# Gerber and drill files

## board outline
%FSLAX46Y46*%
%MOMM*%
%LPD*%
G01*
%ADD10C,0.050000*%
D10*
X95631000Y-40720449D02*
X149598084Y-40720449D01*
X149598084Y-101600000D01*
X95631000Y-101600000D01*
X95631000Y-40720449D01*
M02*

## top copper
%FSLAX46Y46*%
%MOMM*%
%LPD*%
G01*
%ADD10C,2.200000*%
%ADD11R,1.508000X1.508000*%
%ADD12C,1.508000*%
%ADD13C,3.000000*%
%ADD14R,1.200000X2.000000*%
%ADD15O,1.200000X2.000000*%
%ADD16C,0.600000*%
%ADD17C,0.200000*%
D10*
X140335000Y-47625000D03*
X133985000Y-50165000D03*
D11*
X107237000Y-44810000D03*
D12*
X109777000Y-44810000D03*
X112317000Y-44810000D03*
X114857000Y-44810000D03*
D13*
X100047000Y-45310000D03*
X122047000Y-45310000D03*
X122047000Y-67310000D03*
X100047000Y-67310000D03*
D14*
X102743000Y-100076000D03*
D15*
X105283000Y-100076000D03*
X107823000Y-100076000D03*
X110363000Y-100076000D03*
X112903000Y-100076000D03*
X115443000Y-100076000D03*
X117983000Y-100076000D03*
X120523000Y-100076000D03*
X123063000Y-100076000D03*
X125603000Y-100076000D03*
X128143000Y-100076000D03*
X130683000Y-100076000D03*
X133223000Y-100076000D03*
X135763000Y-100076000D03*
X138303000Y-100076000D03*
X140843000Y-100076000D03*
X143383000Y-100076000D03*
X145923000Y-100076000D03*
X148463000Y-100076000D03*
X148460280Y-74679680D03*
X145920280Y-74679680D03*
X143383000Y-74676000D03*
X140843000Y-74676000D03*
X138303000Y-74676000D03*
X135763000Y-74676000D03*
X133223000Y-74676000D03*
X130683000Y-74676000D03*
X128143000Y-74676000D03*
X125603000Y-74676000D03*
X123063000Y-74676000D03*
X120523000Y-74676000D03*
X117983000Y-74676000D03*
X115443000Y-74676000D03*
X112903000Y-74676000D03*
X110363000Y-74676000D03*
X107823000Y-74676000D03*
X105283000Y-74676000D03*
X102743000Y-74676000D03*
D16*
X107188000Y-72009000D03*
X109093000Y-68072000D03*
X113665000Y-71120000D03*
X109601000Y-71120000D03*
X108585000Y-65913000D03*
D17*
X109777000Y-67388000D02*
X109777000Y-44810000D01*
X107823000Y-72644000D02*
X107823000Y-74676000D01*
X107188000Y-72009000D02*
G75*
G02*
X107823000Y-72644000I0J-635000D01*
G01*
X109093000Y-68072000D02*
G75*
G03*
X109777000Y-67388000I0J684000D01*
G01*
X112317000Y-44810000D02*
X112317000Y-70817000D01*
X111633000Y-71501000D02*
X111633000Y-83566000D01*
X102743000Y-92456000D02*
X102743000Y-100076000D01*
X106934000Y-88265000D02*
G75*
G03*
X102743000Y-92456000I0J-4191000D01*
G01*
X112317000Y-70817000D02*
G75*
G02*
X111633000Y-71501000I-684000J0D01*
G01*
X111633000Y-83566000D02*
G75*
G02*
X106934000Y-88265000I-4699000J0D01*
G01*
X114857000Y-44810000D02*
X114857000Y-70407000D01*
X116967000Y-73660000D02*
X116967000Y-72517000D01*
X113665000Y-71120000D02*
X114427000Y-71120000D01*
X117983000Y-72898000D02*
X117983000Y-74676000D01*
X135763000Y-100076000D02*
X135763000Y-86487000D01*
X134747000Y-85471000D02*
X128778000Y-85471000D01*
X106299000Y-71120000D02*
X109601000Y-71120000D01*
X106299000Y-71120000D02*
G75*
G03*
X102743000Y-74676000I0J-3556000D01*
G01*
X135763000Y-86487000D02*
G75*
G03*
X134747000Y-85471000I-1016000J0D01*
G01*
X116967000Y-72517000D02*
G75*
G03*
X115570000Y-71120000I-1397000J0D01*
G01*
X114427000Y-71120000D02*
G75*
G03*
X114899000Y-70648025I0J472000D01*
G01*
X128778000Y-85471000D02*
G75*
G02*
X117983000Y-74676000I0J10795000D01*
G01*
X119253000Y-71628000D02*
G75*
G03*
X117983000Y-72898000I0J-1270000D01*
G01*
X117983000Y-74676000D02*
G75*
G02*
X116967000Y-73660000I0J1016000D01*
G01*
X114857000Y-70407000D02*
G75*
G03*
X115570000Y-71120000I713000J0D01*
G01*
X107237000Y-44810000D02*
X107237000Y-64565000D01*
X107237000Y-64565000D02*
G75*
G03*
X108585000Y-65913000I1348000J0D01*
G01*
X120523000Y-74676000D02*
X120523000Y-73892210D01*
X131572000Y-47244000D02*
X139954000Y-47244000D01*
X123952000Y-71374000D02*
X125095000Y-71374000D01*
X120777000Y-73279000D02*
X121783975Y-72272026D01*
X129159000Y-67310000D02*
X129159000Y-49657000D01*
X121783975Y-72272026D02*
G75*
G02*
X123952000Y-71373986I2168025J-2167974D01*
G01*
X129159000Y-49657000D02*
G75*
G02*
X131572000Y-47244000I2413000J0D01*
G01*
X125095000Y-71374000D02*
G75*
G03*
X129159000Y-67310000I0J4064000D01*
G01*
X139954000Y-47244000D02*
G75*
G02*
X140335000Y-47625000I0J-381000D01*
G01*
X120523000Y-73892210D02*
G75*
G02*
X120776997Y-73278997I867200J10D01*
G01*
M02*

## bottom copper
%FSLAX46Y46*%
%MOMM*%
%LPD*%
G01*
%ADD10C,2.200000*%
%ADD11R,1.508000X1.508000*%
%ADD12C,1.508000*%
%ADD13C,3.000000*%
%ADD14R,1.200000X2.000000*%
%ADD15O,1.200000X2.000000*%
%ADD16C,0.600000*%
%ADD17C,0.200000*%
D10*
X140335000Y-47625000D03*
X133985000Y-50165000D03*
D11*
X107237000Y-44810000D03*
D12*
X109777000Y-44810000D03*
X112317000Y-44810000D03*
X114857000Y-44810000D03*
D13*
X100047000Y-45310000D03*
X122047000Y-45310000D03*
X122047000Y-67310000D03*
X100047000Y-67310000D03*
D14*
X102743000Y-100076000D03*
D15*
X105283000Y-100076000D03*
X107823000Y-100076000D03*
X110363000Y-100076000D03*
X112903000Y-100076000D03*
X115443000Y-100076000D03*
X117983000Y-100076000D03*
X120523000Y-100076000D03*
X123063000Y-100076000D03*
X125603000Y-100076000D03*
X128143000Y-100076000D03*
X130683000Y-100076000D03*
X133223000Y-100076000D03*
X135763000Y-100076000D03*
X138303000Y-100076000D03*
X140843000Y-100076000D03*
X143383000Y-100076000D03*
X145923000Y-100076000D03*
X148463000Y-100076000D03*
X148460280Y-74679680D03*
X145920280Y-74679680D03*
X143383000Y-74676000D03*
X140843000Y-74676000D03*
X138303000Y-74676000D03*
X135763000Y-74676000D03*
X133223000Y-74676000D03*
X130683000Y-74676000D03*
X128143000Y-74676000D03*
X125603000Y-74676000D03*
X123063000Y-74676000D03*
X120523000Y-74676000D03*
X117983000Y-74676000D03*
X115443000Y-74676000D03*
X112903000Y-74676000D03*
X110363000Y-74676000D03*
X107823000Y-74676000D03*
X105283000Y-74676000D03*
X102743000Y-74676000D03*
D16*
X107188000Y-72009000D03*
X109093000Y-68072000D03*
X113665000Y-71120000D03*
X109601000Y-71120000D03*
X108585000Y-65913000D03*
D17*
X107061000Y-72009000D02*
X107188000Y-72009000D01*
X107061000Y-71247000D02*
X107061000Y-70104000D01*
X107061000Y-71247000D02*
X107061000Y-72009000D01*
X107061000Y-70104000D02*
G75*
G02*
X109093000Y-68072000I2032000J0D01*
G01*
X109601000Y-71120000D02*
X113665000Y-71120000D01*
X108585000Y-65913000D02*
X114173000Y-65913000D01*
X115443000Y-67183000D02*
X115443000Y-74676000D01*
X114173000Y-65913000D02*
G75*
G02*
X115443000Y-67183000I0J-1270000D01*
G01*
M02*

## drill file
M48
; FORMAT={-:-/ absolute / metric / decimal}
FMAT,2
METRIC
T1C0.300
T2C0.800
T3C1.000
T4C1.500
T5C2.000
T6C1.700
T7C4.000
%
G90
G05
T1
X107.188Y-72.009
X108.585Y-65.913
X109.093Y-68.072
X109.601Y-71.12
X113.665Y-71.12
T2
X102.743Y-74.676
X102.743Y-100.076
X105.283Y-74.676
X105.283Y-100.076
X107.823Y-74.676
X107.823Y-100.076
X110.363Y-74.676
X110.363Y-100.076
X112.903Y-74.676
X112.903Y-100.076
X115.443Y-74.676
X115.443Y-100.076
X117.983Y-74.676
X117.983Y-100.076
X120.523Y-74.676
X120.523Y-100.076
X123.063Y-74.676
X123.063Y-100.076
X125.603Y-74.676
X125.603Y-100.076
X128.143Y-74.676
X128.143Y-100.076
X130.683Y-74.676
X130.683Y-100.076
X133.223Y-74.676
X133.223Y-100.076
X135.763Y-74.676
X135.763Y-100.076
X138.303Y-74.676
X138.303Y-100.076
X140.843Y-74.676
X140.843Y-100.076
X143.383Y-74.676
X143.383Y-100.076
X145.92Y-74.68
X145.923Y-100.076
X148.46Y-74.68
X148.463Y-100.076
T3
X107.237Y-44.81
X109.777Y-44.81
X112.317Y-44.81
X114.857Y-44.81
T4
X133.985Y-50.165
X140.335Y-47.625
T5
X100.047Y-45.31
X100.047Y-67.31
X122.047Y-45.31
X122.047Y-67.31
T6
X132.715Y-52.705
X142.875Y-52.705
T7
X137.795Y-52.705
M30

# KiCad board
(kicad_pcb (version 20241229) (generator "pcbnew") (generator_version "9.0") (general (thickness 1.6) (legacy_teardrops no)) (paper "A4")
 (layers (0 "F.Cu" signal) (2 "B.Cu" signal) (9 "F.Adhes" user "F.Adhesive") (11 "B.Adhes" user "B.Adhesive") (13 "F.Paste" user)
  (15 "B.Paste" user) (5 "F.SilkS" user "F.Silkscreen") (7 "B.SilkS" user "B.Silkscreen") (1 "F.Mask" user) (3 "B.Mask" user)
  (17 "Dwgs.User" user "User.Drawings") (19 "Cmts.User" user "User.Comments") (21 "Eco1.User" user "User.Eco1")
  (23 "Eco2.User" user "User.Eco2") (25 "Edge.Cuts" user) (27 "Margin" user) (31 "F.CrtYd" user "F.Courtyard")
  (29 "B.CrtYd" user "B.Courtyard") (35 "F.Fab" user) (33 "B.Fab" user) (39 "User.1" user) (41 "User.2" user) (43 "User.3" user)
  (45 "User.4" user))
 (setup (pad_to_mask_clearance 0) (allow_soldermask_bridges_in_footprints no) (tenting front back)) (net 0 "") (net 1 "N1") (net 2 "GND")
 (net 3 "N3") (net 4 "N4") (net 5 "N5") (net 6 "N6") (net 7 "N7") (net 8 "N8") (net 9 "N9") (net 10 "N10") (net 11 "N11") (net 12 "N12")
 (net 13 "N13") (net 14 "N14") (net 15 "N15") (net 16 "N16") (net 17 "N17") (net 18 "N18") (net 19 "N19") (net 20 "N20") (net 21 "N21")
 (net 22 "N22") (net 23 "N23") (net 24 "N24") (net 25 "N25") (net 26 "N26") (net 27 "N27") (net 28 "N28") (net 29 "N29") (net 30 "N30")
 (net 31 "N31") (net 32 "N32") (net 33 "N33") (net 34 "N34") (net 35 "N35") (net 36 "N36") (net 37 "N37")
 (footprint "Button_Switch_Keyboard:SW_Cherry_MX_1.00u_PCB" (layer "F.Cu") (at 140.335 47.625)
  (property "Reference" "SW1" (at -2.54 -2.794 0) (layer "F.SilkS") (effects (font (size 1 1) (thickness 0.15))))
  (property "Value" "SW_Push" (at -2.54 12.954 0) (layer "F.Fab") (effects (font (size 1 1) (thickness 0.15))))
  (pad "" np_thru_hole circle (at -7.62 5.08) (size 1.7 1.7) (drill 1.7) (layers "*.Cu" "*.Mask"))
  (pad "" np_thru_hole circle (at -2.54 5.08) (size 4 4) (drill 4) (layers "*.Cu" "*.Mask"))
  (pad "" np_thru_hole circle (at 2.54 5.08) (size 1.7 1.7) (drill 1.7) (layers "*.Cu" "*.Mask"))
  (pad "1" thru_hole circle (at 0 0) (size 2.2 2.2) (drill 1.5) (layers "*.Cu" "*.Mask") (remove_unused_layers no) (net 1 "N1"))
  (pad "2" thru_hole circle (at -6.35 2.54) (size 2.2 2.2) (drill 1.5) (layers "*.Cu" "*.Mask") (remove_unused_layers no) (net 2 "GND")))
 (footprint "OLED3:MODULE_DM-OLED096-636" (layer "F.Cu") (at 111.047 56.31)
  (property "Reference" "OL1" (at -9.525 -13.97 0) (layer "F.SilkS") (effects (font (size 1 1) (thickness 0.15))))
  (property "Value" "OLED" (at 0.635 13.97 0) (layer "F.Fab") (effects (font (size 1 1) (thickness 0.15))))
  (pad "1" thru_hole rect (at -3.81 -11.5) (size 1.508 1.508) (drill 1) (layers "*.Cu" "*.Mask") (remove_unused_layers no) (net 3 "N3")
   (solder_mask_margin 0.102))
  (pad "2" thru_hole circle (at -1.27 -11.5) (size 1.508 1.508) (drill 1) (layers "*.Cu" "*.Mask") (remove_unused_layers no) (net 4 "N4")
   (solder_mask_margin 0.102))
  (pad "3" thru_hole circle (at 1.27 -11.5) (size 1.508 1.508) (drill 1) (layers "*.Cu" "*.Mask") (remove_unused_layers no) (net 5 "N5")
   (solder_mask_margin 0.102))
  (pad "4" thru_hole circle (at 3.81 -11.5) (size 1.508 1.508) (drill 1) (layers "*.Cu" "*.Mask") (remove_unused_layers no) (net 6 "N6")
   (solder_mask_margin 0.102))
  (pad "S1" thru_hole circle (at -11 -11) (size 3 3) (drill 2) (layers "*.Cu" "*.Mask") (remove_unused_layers no) (solder_mask_margin 0.102))
  (pad "S2" thru_hole circle (at 11 -11) (size 3 3) (drill 2) (layers "*.Cu" "*.Mask") (remove_unused_layers no) (solder_mask_margin 0.102))
  (pad "S3" thru_hole circle (at 11 11) (size 3 3) (drill 2) (layers "*.Cu" "*.Mask") (remove_unused_layers no) (solder_mask_margin 0.102))
  (pad "S4" thru_hole circle (at -11 11) (size 3 3) (drill 2) (layers "*.Cu" "*.Mask") (remove_unused_layers no) (solder_mask_margin 0.102)))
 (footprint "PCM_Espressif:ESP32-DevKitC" (layer "F.Cu") (at 102.743 100.076 90)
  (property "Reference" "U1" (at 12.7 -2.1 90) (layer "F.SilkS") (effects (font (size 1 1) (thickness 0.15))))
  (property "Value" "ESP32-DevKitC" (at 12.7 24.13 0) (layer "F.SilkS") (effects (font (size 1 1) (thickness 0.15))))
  (pad "1" thru_hole rect (at 0 0) (size 1.2 2) (drill 0.8) (layers "*.Cu" "*.Mask") (remove_unused_layers no) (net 5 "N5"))
  (pad "2" thru_hole oval (at 0 2.54) (size 1.2 2) (drill 0.8) (layers "*.Cu" "*.Mask") (remove_unused_layers no) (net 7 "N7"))
  (pad "3" thru_hole oval (at 0 5.08) (size 1.2 2) (drill 0.8) (layers "*.Cu" "*.Mask") (remove_unused_layers no) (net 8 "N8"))
  (pad "4" thru_hole oval (at 0 7.62) (size 1.2 2) (drill 0.8) (layers "*.Cu" "*.Mask") (remove_unused_layers no) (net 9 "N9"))
  (pad "5" thru_hole oval (at 0 10.16) (size 1.2 2) (drill 0.8) (layers "*.Cu" "*.Mask") (remove_unused_layers no) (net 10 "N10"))
  (pad "6" thru_hole oval (at 0 12.7) (size 1.2 2) (drill 0.8) (layers "*.Cu" "*.Mask") (remove_unused_layers no) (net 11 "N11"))
  (pad "7" thru_hole oval (at 0 15.24) (size 1.2 2) (drill 0.8) (layers "*.Cu" "*.Mask") (remove_unused_layers no) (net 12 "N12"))
  (pad "8" thru_hole oval (at 0 17.78) (size 1.2 2) (drill 0.8) (layers "*.Cu" "*.Mask") (remove_unused_layers no) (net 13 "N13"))
  (pad "9" thru_hole oval (at 0 20.32) (size 1.2 2) (drill 0.8) (layers "*.Cu" "*.Mask") (remove_unused_layers no) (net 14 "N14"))
  (pad "10" thru_hole oval (at 0 22.86) (size 1.2 2) (drill 0.8) (layers "*.Cu" "*.Mask") (remove_unused_layers no) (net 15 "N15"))
  (pad "11" thru_hole oval (at 0 25.4) (size 1.2 2) (drill 0.8) (layers "*.Cu" "*.Mask") (remove_unused_layers no) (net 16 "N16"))
  (pad "12" thru_hole oval (at 0 27.94) (size 1.2 2) (drill 0.8) (layers "*.Cu" "*.Mask") (remove_unused_layers no) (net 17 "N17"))
  (pad "13" thru_hole oval (at 0 30.48) (size 1.2 2) (drill 0.8) (layers "*.Cu" "*.Mask") (remove_unused_layers no) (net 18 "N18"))
  (pad "14" thru_hole oval (at 0 33.02) (size 1.2 2) (drill 0.8) (layers "*.Cu" "*.Mask") (remove_unused_layers no) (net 6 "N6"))
  (pad "15" thru_hole oval (at 0 35.56) (size 1.2 2) (drill 0.8) (layers "*.Cu" "*.Mask") (remove_unused_layers no) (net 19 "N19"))
  (pad "16" thru_hole oval (at 0 38.1) (size 1.2 2) (drill 0.8) (layers "*.Cu" "*.Mask") (remove_unused_layers no) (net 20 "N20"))
  (pad "17" thru_hole oval (at 0 40.64) (size 1.2 2) (drill 0.8) (layers "*.Cu" "*.Mask") (remove_unused_layers no) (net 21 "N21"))
  (pad "18" thru_hole oval (at 0 43.18) (size 1.2 2) (drill 0.8) (layers "*.Cu" "*.Mask") (remove_unused_layers no) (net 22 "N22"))
  (pad "19" thru_hole oval (at 0 45.72) (size 1.2 2) (drill 0.8) (layers "*.Cu" "*.Mask") (remove_unused_layers no) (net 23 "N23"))
  (pad "20" thru_hole oval (at 25.39632 45.71728) (size 1.2 2) (drill 0.8) (layers "*.Cu" "*.Mask") (remove_unused_layers no) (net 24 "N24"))
  (pad "21" thru_hole oval (at 25.39632 43.17728) (size 1.2 2) (drill 0.8) (layers "*.Cu" "*.Mask") (remove_unused_layers no) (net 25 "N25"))
  (pad "22" thru_hole oval (at 25.4 40.64) (size 1.2 2) (drill 0.8) (layers "*.Cu" "*.Mask") (remove_unused_layers no) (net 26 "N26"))
  (pad "23" thru_hole oval (at 25.4 38.1) (size 1.2 2) (drill 0.8) (layers "*.Cu" "*.Mask") (remove_unused_layers no) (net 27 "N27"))
  (pad "24" thru_hole oval (at 25.4 35.56) (size 1.2 2) (drill 0.8) (layers "*.Cu" "*.Mask") (remove_unused_layers no) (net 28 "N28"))
  (pad "25" thru_hole oval (at 25.4 33.02) (size 1.2 2) (drill 0.8) (layers "*.Cu" "*.Mask") (remove_unused_layers no) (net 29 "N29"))
  (pad "26" thru_hole oval (at 25.4 30.48) (size 1.2 2) (drill 0.8) (layers "*.Cu" "*.Mask") (remove_unused_layers no) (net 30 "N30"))
  (pad "27" thru_hole oval (at 25.4 27.94) (size 1.2 2) (drill 0.8) (layers "*.Cu" "*.Mask") (remove_unused_layers no) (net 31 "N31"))
  (pad "28" thru_hole oval (at 25.4 25.4) (size 1.2 2) (drill 0.8) (layers "*.Cu" "*.Mask") (remove_unused_layers no) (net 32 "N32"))
  (pad "29" thru_hole oval (at 25.4 22.86) (size 1.2 2) (drill 0.8) (layers "*.Cu" "*.Mask") (remove_unused_layers no) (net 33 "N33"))
  (pad "30" thru_hole oval (at 25.4 20.32) (size 1.2 2) (drill 0.8) (layers "*.Cu" "*.Mask") (remove_unused_layers no) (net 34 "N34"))
  (pad "31" thru_hole oval (at 25.4 17.78) (size 1.2 2) (drill 0.8) (layers "*.Cu" "*.Mask") (remove_unused_layers no) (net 1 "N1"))
  (pad "32" thru_hole oval (at 25.4 15.24) (size 1.2 2) (drill 0.8) (layers "*.Cu" "*.Mask") (remove_unused_layers no) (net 6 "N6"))
  (pad "33" thru_hole oval (at 25.4 12.7) (size 1.2 2) (drill 0.8) (layers "*.Cu" "*.Mask") (remove_unused_layers no) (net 3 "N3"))
  (pad "34" thru_hole oval (at 25.4 10.16) (size 1.2 2) (drill 0.8) (layers "*.Cu" "*.Mask") (remove_unused_layers no) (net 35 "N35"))
  (pad "35" thru_hole oval (at 25.4 7.62) (size 1.2 2) (drill 0.8) (layers "*.Cu" "*.Mask") (remove_unused_layers no) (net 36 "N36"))
  (pad "36" thru_hole oval (at 25.4 5.08) (size 1.2 2) (drill 0.8) (layers "*.Cu" "*.Mask") (remove_unused_layers no) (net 4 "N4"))
  (pad "37" thru_hole oval (at 25.4 2.54) (size 1.2 2) (drill 0.8) (layers "*.Cu" "*.Mask") (remove_unused_layers no) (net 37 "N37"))
  (pad "38" thru_hole oval (at 25.4 0) (size 1.2 2) (drill 0.8) (layers "*.Cu" "*.Mask") (remove_unused_layers no) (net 6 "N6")))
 (gr_rect (start 95.631 40.720449) (end 149.598084 101.6) (stroke (width 0.05) (type default)) (fill no) (layer "Edge.Cuts"))
 (segment (start 109.777 67.388) (end 109.777 44.81) (width 0.2) (layer "F.Cu") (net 4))
 (segment (start 107.823 72.644) (end 107.823 74.676) (width 0.2) (layer "F.Cu") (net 4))
 (via (at 107.188 72.009) (size 0.6) (drill 0.3) (layers "F.Cu" "B.Cu") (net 4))
 (via (at 109.093 68.072) (size 0.6) (drill 0.3) (layers "F.Cu" "B.Cu") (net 4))
 (arc (start 107.188 72.009) (mid 107.637013 72.194987) (end 107.823 72.644) (width 0.2) (layer "F.Cu") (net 4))
 (arc (start 109.093 68.072) (mid 109.576661 67.871661) (end 109.777 67.388) (width 0.2) (layer "F.Cu") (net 4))
 (segment (start 107.061 72.009) (end 107.188 72.009) (width 0.2) (layer "B.Cu") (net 4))
 (segment (start 107.061 71.247) (end 107.061 70.104) (width 0.2) (layer "B.Cu") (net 4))
 (segment (start 107.061 71.247) (end 107.061 72.009) (width 0.2) (layer "B.Cu") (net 4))
 (arc (start 107.061 70.104) (mid 107.656159 68.667159) (end 109.093 68.072) (width 0.2) (layer "B.Cu") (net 4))
 (segment (start 112.317 44.81) (end 112.317 70.817) (width 0.2) (layer "F.Cu") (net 5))
 (segment (start 111.633 71.501) (end 111.633 83.566) (width 0.2) (layer "F.Cu") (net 5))
 (segment (start 102.743 92.456) (end 102.743 100.076) (width 0.2) (layer "F.Cu") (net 5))
 (arc (start 106.934 88.265) (mid 103.970515 89.492515) (end 102.743 92.456) (width 0.2) (layer "F.Cu") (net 5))
 (arc (start 112.317 70.817) (mid 112.116661 71.300661) (end 111.633 71.501) (width 0.2) (layer "F.Cu") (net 5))
 (arc (start 111.633 83.566) (mid 110.256695 86.888695) (end 106.934 88.265) (width 0.2) (layer "F.Cu") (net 5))
 (segment (start 114.857 44.81) (end 114.857 70.407) (width 0.2) (layer "F.Cu") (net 6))
 (segment (start 116.967 73.66) (end 116.967 72.517) (width 0.2) (layer "F.Cu") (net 6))
 (segment (start 113.665 71.12) (end 114.427 71.12) (width 0.2) (layer "F.Cu") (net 6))
 (segment (start 117.983 72.898) (end 117.983 74.676) (width 0.2) (layer "F.Cu") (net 6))
 (segment (start 135.763 100.076) (end 135.763 86.487) (width 0.2) (layer "F.Cu") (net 6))
 (segment (start 134.747 85.471) (end 128.778 85.471) (width 0.2) (layer "F.Cu") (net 6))
 (segment (start 106.299 71.12) (end 109.601 71.12) (width 0.2) (layer "F.Cu") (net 6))
 (via (at 113.665 71.12) (size 0.6) (drill 0.3) (layers "F.Cu" "B.Cu") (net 6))
 (via (at 109.601 71.12) (size 0.6) (drill 0.3) (layers "F.Cu" "B.Cu") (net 6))
 (arc (start 106.299 71.12) (mid 103.784528 72.161528) (end 102.743 74.676) (width 0.2) (layer "F.Cu") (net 6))
 (arc (start 135.763 86.487) (mid 135.46542 85.76858) (end 134.747 85.471) (width 0.2) (layer "F.Cu") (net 6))
 (arc (start 116.967 72.517) (mid 116.557828 71.529172) (end 115.57 71.12) (width 0.2) (layer "F.Cu") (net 6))
 (arc (start 114.427 71.12) (mid 114.760737 70.981762) (end 114.898975 70.648025) (width 0.2) (layer "F.Cu") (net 6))
 (arc (start 128.778 85.471) (mid 121.144782 82.309218) (end 117.983 74.676) (width 0.2) (layer "F.Cu") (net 6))
 (arc (start 119.253 71.628) (mid 118.354974 71.999974) (end 117.983 72.898) (width 0.2) (layer "F.Cu") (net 6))
 (arc (start 117.983 74.676) (mid 117.26458 74.37842) (end 116.967 73.66) (width 0.2) (layer "F.Cu") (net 6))
 (arc (start 114.857 70.407) (mid 115.065833 70.911167) (end 115.57 71.12) (width 0.2) (layer "F.Cu") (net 6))
 (segment (start 109.601 71.12) (end 113.665 71.12) (width 0.2) (layer "B.Cu") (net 6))
 (segment (start 107.237 44.81) (end 107.237 64.565) (width 0.2) (layer "F.Cu") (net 3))
 (via (at 108.585 65.913) (size 0.6) (drill 0.3) (layers "F.Cu" "B.Cu") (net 3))
 (arc (start 107.237 64.565) (mid 107.63182 65.51818) (end 108.585 65.913) (width 0.2) (layer "F.Cu") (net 3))
 (segment (start 108.585 65.913) (end 114.173 65.913) (width 0.2) (layer "B.Cu") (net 3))
 (segment (start 115.443 67.183) (end 115.443 74.676) (width 0.2) (layer "B.Cu") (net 3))
 (arc (start 114.173 65.913) (mid 115.071026 66.284974) (end 115.443 67.183) (width 0.2) (layer "B.Cu") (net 3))
 (segment (start 120.523 74.676) (end 120.523 73.89221) (width 0.2) (layer "F.Cu") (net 1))
 (segment (start 131.572 47.244) (end 139.954 47.244) (width 0.2) (layer "F.Cu") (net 1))
 (segment (start 123.952 71.374) (end 125.095 71.374) (width 0.2) (layer "F.Cu") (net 1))
 (segment (start 120.777 73.279) (end 121.783975 72.272026) (width 0.2) (layer "F.Cu") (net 1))
 (segment (start 129.159 67.31) (end 129.159 49.657) (width 0.2) (layer "F.Cu") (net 1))
 (arc (start 121.783975 72.272026) (mid 122.778673 71.607389) (end 123.952 71.374) (width 0.2) (layer "F.Cu") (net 1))
 (arc (start 129.159 49.657) (mid 129.865751 47.950751) (end 131.572 47.244) (width 0.2) (layer "F.Cu") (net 1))
 (arc (start 125.095 71.374) (mid 127.968682 70.183682) (end 129.159 67.31) (width 0.2) (layer "F.Cu") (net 1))
 (arc (start 139.954 47.244) (mid 140.223408 47.355592) (end 140.335 47.625) (width 0.2) (layer "F.Cu") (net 1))
 (arc (start 120.523 73.89221) (mid 120.589012 73.560343) (end 120.777 73.279) (width 0.2) (layer "F.Cu") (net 1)))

